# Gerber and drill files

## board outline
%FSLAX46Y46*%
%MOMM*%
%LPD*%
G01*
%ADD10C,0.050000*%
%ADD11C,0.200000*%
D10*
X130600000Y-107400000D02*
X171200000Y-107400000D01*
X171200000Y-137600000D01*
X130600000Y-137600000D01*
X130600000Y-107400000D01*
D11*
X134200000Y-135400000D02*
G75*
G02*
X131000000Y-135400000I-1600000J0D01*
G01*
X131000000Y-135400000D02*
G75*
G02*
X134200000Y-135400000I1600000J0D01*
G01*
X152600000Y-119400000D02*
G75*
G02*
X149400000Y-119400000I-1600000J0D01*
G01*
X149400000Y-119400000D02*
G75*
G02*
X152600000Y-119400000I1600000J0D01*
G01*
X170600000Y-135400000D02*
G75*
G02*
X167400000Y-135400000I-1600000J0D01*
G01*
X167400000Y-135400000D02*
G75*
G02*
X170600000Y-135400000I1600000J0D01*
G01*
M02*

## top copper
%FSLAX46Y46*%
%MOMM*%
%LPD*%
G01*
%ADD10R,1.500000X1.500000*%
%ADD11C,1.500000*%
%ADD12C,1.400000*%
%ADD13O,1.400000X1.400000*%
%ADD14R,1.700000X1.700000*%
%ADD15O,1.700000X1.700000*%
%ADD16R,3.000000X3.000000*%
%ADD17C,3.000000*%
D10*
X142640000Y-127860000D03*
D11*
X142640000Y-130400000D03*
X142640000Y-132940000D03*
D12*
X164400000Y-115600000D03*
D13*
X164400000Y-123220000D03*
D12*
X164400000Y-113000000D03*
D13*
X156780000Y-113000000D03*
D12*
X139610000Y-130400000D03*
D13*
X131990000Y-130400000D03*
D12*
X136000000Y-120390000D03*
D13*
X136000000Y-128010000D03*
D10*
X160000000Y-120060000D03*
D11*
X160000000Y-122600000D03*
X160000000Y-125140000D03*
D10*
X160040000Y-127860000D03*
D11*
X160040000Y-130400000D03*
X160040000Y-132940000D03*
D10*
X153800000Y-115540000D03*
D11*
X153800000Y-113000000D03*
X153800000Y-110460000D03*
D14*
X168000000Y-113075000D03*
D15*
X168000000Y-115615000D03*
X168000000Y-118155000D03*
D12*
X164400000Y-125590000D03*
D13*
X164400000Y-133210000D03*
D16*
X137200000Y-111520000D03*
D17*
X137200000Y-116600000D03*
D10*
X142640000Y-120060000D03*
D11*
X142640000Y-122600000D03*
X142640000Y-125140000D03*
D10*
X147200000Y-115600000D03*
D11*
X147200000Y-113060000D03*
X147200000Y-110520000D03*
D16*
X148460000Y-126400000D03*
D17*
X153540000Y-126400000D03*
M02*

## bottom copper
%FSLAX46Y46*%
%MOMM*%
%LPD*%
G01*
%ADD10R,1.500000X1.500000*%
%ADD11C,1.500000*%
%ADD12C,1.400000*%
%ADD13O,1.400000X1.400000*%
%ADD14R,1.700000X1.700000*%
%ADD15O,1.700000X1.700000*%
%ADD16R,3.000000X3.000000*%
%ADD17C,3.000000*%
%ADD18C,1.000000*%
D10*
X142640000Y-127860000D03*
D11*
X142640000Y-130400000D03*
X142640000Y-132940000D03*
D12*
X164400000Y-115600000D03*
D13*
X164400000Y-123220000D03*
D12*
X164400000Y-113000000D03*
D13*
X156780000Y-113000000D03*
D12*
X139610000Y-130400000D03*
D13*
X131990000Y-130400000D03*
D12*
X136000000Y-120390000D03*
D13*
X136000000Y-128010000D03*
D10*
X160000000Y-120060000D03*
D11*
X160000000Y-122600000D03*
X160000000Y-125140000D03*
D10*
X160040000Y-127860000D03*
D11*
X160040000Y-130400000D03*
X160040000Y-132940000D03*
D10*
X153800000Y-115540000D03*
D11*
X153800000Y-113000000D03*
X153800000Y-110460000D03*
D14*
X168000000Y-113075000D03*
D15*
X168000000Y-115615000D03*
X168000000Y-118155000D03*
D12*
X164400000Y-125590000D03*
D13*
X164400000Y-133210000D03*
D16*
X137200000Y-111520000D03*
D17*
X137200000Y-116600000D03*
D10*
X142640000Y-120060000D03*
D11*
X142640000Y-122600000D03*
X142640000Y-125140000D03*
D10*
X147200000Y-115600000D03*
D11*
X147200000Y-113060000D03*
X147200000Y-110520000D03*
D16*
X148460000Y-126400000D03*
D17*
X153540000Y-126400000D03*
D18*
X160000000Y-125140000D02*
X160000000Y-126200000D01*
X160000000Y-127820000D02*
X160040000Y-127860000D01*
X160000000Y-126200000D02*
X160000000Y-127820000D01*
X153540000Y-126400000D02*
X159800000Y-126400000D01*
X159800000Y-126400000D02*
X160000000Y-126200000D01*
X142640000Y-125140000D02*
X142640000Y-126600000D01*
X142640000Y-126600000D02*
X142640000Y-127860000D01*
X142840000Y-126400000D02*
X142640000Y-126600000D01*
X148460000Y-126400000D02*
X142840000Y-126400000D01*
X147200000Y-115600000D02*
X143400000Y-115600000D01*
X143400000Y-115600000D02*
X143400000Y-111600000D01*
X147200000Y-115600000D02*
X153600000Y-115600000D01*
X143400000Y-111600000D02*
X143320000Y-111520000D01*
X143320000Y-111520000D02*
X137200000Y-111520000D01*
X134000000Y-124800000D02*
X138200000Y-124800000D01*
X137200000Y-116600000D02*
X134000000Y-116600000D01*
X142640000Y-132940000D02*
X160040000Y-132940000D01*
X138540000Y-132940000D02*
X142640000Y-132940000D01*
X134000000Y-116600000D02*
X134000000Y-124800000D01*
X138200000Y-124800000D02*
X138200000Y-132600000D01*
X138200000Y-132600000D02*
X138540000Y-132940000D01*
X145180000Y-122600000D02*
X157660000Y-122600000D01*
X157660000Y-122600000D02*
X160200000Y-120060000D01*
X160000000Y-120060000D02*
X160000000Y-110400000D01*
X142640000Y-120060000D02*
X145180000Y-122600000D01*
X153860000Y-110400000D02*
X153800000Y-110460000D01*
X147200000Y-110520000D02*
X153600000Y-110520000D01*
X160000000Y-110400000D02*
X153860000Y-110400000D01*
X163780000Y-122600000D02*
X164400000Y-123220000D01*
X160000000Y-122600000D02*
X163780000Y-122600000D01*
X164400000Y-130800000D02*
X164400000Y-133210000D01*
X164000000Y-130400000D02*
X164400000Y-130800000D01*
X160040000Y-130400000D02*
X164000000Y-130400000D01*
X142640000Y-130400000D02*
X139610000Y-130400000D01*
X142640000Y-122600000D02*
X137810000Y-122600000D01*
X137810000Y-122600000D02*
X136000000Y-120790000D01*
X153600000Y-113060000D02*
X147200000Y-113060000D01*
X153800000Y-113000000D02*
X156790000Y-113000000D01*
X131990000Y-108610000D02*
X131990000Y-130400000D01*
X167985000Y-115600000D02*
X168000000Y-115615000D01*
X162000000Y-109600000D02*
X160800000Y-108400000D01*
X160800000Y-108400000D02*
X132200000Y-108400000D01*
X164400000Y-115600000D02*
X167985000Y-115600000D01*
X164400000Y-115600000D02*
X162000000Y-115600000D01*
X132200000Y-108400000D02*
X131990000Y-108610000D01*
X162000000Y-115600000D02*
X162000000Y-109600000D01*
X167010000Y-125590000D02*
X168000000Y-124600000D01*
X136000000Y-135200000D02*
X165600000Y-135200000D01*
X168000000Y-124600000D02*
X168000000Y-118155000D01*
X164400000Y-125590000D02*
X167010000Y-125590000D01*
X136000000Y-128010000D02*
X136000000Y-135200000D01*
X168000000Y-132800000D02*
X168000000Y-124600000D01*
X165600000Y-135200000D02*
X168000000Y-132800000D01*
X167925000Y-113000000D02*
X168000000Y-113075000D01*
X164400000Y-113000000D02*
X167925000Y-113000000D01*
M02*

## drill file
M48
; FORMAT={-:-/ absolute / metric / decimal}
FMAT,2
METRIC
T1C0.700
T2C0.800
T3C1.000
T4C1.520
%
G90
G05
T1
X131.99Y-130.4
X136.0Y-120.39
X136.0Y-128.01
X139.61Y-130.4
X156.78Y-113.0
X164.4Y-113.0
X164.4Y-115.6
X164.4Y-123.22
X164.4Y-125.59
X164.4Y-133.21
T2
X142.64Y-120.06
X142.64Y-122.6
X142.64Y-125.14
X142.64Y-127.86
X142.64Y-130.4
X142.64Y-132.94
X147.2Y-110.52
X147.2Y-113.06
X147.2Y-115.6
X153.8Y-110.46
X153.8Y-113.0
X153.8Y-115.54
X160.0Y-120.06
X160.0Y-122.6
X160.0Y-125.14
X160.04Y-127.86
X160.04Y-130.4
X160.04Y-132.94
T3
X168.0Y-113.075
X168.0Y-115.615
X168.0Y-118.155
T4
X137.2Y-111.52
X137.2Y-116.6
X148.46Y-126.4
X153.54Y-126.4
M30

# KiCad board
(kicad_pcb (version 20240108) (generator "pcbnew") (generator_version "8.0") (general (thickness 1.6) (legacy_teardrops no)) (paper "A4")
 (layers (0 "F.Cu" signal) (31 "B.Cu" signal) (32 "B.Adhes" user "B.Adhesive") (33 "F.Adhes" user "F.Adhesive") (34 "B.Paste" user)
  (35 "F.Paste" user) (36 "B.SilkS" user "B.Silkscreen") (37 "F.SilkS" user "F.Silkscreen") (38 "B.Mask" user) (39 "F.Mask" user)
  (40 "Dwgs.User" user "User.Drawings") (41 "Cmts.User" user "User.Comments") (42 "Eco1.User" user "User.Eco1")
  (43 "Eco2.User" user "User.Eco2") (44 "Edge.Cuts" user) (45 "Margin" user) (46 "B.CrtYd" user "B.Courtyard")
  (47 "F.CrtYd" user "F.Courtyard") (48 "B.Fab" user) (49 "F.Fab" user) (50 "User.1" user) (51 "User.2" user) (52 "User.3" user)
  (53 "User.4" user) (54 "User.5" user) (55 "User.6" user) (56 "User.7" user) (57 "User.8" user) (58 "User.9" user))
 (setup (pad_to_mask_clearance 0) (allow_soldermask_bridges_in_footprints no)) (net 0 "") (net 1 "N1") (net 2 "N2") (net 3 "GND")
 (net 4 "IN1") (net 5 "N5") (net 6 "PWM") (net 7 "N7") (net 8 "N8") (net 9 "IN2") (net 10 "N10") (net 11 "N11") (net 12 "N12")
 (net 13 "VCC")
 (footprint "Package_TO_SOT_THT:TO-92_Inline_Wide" (layer "F.Cu") (at 142.64 127.86 -90)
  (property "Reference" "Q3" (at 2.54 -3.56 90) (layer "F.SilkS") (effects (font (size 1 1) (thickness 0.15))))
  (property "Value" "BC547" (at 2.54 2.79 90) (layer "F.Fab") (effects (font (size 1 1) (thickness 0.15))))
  (pad "1" thru_hole rect (at 0 0 270) (size 1.5 1.5) (drill 0.8) (layers "*.Cu" "*.Mask") (remove_unused_layers no) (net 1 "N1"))
  (pad "2" thru_hole circle (at 2.54 0 270) (size 1.5 1.5) (drill 0.8) (layers "*.Cu" "*.Mask") (remove_unused_layers no) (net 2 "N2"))
  (pad "3" thru_hole circle (at 5.08 0 270) (size 1.5 1.5) (drill 0.8) (layers "*.Cu" "*.Mask") (remove_unused_layers no) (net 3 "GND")))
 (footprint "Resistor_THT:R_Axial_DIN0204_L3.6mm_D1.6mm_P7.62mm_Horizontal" (layer "F.Cu") (at 164.4 115.6 -90)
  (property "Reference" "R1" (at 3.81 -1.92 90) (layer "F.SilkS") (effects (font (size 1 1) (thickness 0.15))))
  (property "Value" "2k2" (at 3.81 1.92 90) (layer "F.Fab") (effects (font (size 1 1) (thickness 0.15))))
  (pad "1" thru_hole circle (at 0 0 270) (size 1.4 1.4) (drill 0.7) (layers "*.Cu" "*.Mask") (remove_unused_layers no) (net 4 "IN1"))
  (pad "2" thru_hole oval (at 7.62 0 270) (size 1.4 1.4) (drill 0.7) (layers "*.Cu" "*.Mask") (remove_unused_layers no) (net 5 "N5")))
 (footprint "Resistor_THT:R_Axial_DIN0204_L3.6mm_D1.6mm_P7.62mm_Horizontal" (layer "F.Cu") (at 164.4 113 180)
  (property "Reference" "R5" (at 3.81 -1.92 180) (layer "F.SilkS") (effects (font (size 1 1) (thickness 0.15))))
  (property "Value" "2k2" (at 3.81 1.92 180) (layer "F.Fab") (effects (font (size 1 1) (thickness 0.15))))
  (pad "1" thru_hole circle (at 0 0 180) (size 1.4 1.4) (drill 0.7) (layers "*.Cu" "*.Mask") (remove_unused_layers no) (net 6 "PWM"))
  (pad "2" thru_hole oval (at 7.62 0 180) (size 1.4 1.4) (drill 0.7) (layers "*.Cu" "*.Mask") (remove_unused_layers no) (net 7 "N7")))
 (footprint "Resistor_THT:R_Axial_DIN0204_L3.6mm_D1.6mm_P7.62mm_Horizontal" (layer "F.Cu") (at 139.61 130.4 180)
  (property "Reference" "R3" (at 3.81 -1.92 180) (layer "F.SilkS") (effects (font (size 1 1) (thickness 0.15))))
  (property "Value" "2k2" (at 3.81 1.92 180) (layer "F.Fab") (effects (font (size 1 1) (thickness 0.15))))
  (pad "1" thru_hole circle (at 0 0 180) (size 1.4 1.4) (drill 0.7) (layers "*.Cu" "*.Mask") (remove_unused_layers no) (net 2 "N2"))
  (pad "2" thru_hole oval (at 7.62 0 180) (size 1.4 1.4) (drill 0.7) (layers "*.Cu" "*.Mask") (remove_unused_layers no) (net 4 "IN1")))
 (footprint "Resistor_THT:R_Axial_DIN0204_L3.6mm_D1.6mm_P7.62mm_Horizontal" (layer "F.Cu") (at 136 120.39 -90)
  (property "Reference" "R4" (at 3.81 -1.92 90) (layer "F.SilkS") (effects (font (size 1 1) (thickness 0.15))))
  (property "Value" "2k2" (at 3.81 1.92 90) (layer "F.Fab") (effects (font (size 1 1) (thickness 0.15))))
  (pad "1" thru_hole circle (at 0 0 270) (size 1.4 1.4) (drill 0.7) (layers "*.Cu" "*.Mask") (remove_unused_layers no) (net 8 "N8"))
  (pad "2" thru_hole oval (at 7.62 0 270) (size 1.4 1.4) (drill 0.7) (layers "*.Cu" "*.Mask") (remove_unused_layers no) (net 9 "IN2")))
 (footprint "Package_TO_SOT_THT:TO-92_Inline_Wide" (layer "F.Cu") (at 160 120.06 -90)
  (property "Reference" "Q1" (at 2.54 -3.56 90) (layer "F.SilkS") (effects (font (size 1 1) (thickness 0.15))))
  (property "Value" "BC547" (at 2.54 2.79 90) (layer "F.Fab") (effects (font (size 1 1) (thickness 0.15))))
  (pad "1" thru_hole rect (at 0 0 270) (size 1.5 1.5) (drill 0.8) (layers "*.Cu" "*.Mask") (remove_unused_layers no) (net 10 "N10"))
  (pad "2" thru_hole circle (at 2.54 0 270) (size 1.5 1.5) (drill 0.8) (layers "*.Cu" "*.Mask") (remove_unused_layers no) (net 5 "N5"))
  (pad "3" thru_hole circle (at 5.08 0 270) (size 1.5 1.5) (drill 0.8) (layers "*.Cu" "*.Mask") (remove_unused_layers no) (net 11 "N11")))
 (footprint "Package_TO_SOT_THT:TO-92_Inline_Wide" (layer "F.Cu") (at 160.04 127.86 -90)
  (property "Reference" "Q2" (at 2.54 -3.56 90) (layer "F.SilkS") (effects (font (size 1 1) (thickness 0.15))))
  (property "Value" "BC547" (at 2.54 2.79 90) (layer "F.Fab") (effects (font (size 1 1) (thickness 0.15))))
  (pad "1" thru_hole rect (at 0 0 270) (size 1.5 1.5) (drill 0.8) (layers "*.Cu" "*.Mask") (remove_unused_layers no) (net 11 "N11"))
  (pad "2" thru_hole circle (at 2.54 0 270) (size 1.5 1.5) (drill 0.8) (layers "*.Cu" "*.Mask") (remove_unused_layers no) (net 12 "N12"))
  (pad "3" thru_hole circle (at 5.08 0 270) (size 1.5 1.5) (drill 0.8) (layers "*.Cu" "*.Mask") (remove_unused_layers no) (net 3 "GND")))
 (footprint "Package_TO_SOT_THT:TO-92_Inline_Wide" (layer "F.Cu") (at 153.8 115.54 90)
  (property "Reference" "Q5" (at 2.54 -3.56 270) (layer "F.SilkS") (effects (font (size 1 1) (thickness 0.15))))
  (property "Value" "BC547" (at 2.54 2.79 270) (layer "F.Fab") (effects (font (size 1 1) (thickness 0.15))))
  (pad "1" thru_hole rect (at 0 0 90) (size 1.5 1.5) (drill 0.8) (layers "*.Cu" "*.Mask") (remove_unused_layers no) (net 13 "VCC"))
  (pad "2" thru_hole circle (at 2.54 0 90) (size 1.5 1.5) (drill 0.8) (layers "*.Cu" "*.Mask") (remove_unused_layers no) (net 7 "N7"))
  (pad "3" thru_hole circle (at 5.08 0 90) (size 1.5 1.5) (drill 0.8) (layers "*.Cu" "*.Mask") (remove_unused_layers no) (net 10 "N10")))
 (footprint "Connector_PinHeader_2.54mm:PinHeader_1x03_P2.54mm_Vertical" (layer "F.Cu") (at 168 113.075)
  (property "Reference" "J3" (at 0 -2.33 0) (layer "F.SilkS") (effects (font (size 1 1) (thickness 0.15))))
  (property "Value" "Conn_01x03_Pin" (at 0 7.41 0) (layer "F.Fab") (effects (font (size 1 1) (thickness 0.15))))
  (pad "1" thru_hole rect (at 0 0) (size 1.7 1.7) (drill 1) (layers "*.Cu" "*.Mask") (remove_unused_layers no) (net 6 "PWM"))
  (pad "2" thru_hole oval (at 0 2.54) (size 1.7 1.7) (drill 1) (layers "*.Cu" "*.Mask") (remove_unused_layers no) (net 4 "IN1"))
  (pad "3" thru_hole oval (at 0 5.08) (size 1.7 1.7) (drill 1) (layers "*.Cu" "*.Mask") (remove_unused_layers no) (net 9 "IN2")))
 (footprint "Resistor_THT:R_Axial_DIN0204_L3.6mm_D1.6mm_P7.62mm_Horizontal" (layer "F.Cu") (at 164.4 125.59 -90)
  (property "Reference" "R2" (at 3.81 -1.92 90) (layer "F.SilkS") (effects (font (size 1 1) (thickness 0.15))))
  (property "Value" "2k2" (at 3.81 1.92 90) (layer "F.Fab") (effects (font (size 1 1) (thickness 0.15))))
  (pad "1" thru_hole circle (at 0 0 270) (size 1.4 1.4) (drill 0.7) (layers "*.Cu" "*.Mask") (remove_unused_layers no) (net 9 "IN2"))
  (pad "2" thru_hole oval (at 7.62 0 270) (size 1.4 1.4) (drill 0.7) (layers "*.Cu" "*.Mask") (remove_unused_layers no) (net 12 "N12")))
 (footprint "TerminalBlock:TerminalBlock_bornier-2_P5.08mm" (layer "F.Cu") (at 137.2 111.52 -90)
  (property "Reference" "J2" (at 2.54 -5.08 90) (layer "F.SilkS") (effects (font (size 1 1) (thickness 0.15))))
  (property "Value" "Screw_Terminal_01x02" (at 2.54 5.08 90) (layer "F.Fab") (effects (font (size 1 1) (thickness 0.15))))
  (pad "1" thru_hole rect (at 0 0 270) (size 3 3) (drill 1.52) (layers "*.Cu" "*.Mask") (remove_unused_layers no) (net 13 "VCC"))
  (pad "2" thru_hole circle (at 5.08 0 270) (size 3 3) (drill 1.52) (layers "*.Cu" "*.Mask") (remove_unused_layers no) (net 3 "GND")))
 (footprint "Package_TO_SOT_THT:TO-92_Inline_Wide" (layer "F.Cu") (at 142.64 120.06 -90)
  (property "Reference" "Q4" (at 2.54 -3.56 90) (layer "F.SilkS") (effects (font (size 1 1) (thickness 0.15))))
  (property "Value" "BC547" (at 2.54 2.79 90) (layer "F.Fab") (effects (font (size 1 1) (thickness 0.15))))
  (pad "1" thru_hole rect (at 0 0 270) (size 1.5 1.5) (drill 0.8) (layers "*.Cu" "*.Mask") (remove_unused_layers no) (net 10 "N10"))
  (pad "2" thru_hole circle (at 2.54 0 270) (size 1.5 1.5) (drill 0.8) (layers "*.Cu" "*.Mask") (remove_unused_layers no) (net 8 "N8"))
  (pad "3" thru_hole circle (at 5.08 0 270) (size 1.5 1.5) (drill 0.8) (layers "*.Cu" "*.Mask") (remove_unused_layers no) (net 1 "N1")))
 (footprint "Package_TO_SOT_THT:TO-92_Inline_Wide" (layer "F.Cu") (at 147.2 115.6 90)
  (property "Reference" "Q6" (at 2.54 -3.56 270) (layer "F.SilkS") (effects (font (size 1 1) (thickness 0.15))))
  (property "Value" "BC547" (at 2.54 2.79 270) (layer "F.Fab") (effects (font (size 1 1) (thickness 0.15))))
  (pad "1" thru_hole rect (at 0 0 90) (size 1.5 1.5) (drill 0.8) (layers "*.Cu" "*.Mask") (remove_unused_layers no) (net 13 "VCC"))
  (pad "2" thru_hole circle (at 2.54 0 90) (size 1.5 1.5) (drill 0.8) (layers "*.Cu" "*.Mask") (remove_unused_layers no) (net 7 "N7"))
  (pad "3" thru_hole circle (at 5.08 0 90) (size 1.5 1.5) (drill 0.8) (layers "*.Cu" "*.Mask") (remove_unused_layers no) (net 10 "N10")))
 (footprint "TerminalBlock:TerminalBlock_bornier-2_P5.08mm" (layer "F.Cu") (at 148.46 126.4)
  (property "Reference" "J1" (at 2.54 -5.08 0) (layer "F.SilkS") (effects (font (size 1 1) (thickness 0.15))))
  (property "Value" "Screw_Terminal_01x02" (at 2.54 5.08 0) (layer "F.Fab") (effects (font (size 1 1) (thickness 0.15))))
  (pad "1" thru_hole rect (at 0 0) (size 3 3) (drill 1.52) (layers "*.Cu" "*.Mask") (remove_unused_layers no) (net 1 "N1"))
  (pad "2" thru_hole circle (at 5.08 0) (size 3 3) (drill 1.52) (layers "*.Cu" "*.Mask") (remove_unused_layers no) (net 11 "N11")))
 (gr_rect (start 130.6 107.4) (end 171.2 137.6) (stroke (width 0.05) (type default)) (fill none) (layer "Edge.Cuts"))
 (gr_circle (center 132.6 135.4) (end 134.2 135.4) (stroke (width 0.2) (type default)) (fill none) (layer "Edge.Cuts"))
 (gr_circle (center 151 119.4) (end 152.6 119.4) (stroke (width 0.2) (type default)) (fill none) (layer "Edge.Cuts"))
 (gr_circle (center 169 135.4) (end 170.6 135.4) (stroke (width 0.2) (type default)) (fill none) (layer "Edge.Cuts"))
 (segment (start 160 125.14) (end 160 126.2) (width 1) (layer "B.Cu") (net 11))
 (segment (start 160 127.82) (end 160.04 127.86) (width 1) (layer "B.Cu") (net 11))
 (segment (start 160 126.2) (end 160 127.82) (width 1) (layer "B.Cu") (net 11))
 (segment (start 153.54 126.4) (end 159.8 126.4) (width 1) (layer "B.Cu") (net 11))
 (segment (start 159.8 126.4) (end 160 126.2) (width 1) (layer "B.Cu") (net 11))
 (segment (start 142.64 125.14) (end 142.64 126.6) (width 1) (layer "B.Cu") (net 1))
 (segment (start 142.64 126.6) (end 142.64 127.86) (width 1) (layer "B.Cu") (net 1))
 (segment (start 142.84 126.4) (end 142.64 126.6) (width 1) (layer "B.Cu") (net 1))
 (segment (start 148.46 126.4) (end 142.84 126.4) (width 1) (layer "B.Cu") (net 1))
 (segment (start 147.2 115.6) (end 143.4 115.6) (width 1) (layer "B.Cu") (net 13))
 (segment (start 143.4 115.6) (end 143.4 111.6) (width 1) (layer "B.Cu") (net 13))
 (segment (start 147.2 115.6) (end 153.6 115.6) (width 1) (layer "B.Cu") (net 13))
 (segment (start 143.4 111.6) (end 143.32 111.52) (width 1) (layer "B.Cu") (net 13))
 (segment (start 143.32 111.52) (end 137.2 111.52) (width 1) (layer "B.Cu") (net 13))
 (segment (start 134 124.8) (end 138.2 124.8) (width 1) (layer "B.Cu") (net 3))
 (segment (start 137.2 116.6) (end 134 116.6) (width 1) (layer "B.Cu") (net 3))
 (segment (start 142.64 132.94) (end 160.04 132.94) (width 1) (layer "B.Cu") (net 3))
 (segment (start 138.54 132.94) (end 142.64 132.94) (width 1) (layer "B.Cu") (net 3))
 (segment (start 134 116.6) (end 134 124.8) (width 1) (layer "B.Cu") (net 3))
 (segment (start 138.2 124.8) (end 138.2 132.6) (width 1) (layer "B.Cu") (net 3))
 (segment (start 138.2 132.6) (end 138.54 132.94) (width 1) (layer "B.Cu") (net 3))
 (segment (start 145.18 122.6) (end 157.66 122.6) (width 1) (layer "B.Cu") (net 10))
 (segment (start 157.66 122.6) (end 160.2 120.06) (width 1) (layer "B.Cu") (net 10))
 (segment (start 160 120.06) (end 160 110.4) (width 1) (layer "B.Cu") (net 10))
 (segment (start 142.64 120.06) (end 145.18 122.6) (width 1) (layer "B.Cu") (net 10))
 (segment (start 153.86 110.4) (end 153.8 110.46) (width 1) (layer "B.Cu") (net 10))
 (segment (start 147.2 110.52) (end 153.6 110.52) (width 1) (layer "B.Cu") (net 10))
 (segment (start 160 110.4) (end 153.86 110.4) (width 1) (layer "B.Cu") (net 10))
 (segment (start 163.78 122.6) (end 164.4 123.22) (width 1) (layer "B.Cu") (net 5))
 (segment (start 160 122.6) (end 163.78 122.6) (width 1) (layer "B.Cu") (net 5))
 (segment (start 164.4 130.8) (end 164.4 133.21) (width 1) (layer "B.Cu") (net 12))
 (segment (start 164 130.4) (end 164.4 130.8) (width 1) (layer "B.Cu") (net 12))
 (segment (start 160.04 130.4) (end 164 130.4) (width 1) (layer "B.Cu") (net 12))
 (segment (start 142.64 130.4) (end 139.61 130.4) (width 1) (layer "B.Cu") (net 2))
 (segment (start 142.64 122.6) (end 137.81 122.6) (width 1) (layer "B.Cu") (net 8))
 (segment (start 137.81 122.6) (end 136 120.79) (width 1) (layer "B.Cu") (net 8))
 (segment (start 153.6 113.06) (end 147.2 113.06) (width 1) (layer "B.Cu") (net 7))
 (segment (start 153.8 113) (end 156.79 113) (width 1) (layer "B.Cu") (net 7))
 (segment (start 131.99 108.61) (end 131.99 130.4) (width 1) (layer "B.Cu") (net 4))
 (segment (start 167.985 115.6) (end 168 115.615) (width 1) (layer "B.Cu") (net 4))
 (segment (start 162 109.6) (end 160.8 108.4) (width 1) (layer "B.Cu") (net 4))
 (segment (start 160.8 108.4) (end 132.2 108.4) (width 1) (layer "B.Cu") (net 4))
 (segment (start 164.4 115.6) (end 167.985 115.6) (width 1) (layer "B.Cu") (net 4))
 (segment (start 164.4 115.6) (end 162 115.6) (width 1) (layer "B.Cu") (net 4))
 (segment (start 132.2 108.4) (end 131.99 108.61) (width 1) (layer "B.Cu") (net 4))
 (segment (start 162 115.6) (end 162 109.6) (width 1) (layer "B.Cu") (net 4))
 (segment (start 167.01 125.59) (end 168 124.6) (width 1) (layer "B.Cu") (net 9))
 (segment (start 136 135.2) (end 165.6 135.2) (width 1) (layer "B.Cu") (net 9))
 (segment (start 168 124.6) (end 168 118.155) (width 1) (layer "B.Cu") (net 9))
 (segment (start 164.4 125.59) (end 167.01 125.59) (width 1) (layer "B.Cu") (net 9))
 (segment (start 136 128.01) (end 136 135.2) (width 1) (layer "B.Cu") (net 9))
 (segment (start 168 132.8) (end 168 124.6) (width 1) (layer "B.Cu") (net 9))
 (segment (start 165.6 135.2) (end 168 132.8) (width 1) (layer "B.Cu") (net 9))
 (segment (start 167.925 113) (end 168 113.075) (width 1) (layer "B.Cu") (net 6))
 (segment (start 164.4 113) (end 167.925 113) (width 1) (layer "B.Cu") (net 6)))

